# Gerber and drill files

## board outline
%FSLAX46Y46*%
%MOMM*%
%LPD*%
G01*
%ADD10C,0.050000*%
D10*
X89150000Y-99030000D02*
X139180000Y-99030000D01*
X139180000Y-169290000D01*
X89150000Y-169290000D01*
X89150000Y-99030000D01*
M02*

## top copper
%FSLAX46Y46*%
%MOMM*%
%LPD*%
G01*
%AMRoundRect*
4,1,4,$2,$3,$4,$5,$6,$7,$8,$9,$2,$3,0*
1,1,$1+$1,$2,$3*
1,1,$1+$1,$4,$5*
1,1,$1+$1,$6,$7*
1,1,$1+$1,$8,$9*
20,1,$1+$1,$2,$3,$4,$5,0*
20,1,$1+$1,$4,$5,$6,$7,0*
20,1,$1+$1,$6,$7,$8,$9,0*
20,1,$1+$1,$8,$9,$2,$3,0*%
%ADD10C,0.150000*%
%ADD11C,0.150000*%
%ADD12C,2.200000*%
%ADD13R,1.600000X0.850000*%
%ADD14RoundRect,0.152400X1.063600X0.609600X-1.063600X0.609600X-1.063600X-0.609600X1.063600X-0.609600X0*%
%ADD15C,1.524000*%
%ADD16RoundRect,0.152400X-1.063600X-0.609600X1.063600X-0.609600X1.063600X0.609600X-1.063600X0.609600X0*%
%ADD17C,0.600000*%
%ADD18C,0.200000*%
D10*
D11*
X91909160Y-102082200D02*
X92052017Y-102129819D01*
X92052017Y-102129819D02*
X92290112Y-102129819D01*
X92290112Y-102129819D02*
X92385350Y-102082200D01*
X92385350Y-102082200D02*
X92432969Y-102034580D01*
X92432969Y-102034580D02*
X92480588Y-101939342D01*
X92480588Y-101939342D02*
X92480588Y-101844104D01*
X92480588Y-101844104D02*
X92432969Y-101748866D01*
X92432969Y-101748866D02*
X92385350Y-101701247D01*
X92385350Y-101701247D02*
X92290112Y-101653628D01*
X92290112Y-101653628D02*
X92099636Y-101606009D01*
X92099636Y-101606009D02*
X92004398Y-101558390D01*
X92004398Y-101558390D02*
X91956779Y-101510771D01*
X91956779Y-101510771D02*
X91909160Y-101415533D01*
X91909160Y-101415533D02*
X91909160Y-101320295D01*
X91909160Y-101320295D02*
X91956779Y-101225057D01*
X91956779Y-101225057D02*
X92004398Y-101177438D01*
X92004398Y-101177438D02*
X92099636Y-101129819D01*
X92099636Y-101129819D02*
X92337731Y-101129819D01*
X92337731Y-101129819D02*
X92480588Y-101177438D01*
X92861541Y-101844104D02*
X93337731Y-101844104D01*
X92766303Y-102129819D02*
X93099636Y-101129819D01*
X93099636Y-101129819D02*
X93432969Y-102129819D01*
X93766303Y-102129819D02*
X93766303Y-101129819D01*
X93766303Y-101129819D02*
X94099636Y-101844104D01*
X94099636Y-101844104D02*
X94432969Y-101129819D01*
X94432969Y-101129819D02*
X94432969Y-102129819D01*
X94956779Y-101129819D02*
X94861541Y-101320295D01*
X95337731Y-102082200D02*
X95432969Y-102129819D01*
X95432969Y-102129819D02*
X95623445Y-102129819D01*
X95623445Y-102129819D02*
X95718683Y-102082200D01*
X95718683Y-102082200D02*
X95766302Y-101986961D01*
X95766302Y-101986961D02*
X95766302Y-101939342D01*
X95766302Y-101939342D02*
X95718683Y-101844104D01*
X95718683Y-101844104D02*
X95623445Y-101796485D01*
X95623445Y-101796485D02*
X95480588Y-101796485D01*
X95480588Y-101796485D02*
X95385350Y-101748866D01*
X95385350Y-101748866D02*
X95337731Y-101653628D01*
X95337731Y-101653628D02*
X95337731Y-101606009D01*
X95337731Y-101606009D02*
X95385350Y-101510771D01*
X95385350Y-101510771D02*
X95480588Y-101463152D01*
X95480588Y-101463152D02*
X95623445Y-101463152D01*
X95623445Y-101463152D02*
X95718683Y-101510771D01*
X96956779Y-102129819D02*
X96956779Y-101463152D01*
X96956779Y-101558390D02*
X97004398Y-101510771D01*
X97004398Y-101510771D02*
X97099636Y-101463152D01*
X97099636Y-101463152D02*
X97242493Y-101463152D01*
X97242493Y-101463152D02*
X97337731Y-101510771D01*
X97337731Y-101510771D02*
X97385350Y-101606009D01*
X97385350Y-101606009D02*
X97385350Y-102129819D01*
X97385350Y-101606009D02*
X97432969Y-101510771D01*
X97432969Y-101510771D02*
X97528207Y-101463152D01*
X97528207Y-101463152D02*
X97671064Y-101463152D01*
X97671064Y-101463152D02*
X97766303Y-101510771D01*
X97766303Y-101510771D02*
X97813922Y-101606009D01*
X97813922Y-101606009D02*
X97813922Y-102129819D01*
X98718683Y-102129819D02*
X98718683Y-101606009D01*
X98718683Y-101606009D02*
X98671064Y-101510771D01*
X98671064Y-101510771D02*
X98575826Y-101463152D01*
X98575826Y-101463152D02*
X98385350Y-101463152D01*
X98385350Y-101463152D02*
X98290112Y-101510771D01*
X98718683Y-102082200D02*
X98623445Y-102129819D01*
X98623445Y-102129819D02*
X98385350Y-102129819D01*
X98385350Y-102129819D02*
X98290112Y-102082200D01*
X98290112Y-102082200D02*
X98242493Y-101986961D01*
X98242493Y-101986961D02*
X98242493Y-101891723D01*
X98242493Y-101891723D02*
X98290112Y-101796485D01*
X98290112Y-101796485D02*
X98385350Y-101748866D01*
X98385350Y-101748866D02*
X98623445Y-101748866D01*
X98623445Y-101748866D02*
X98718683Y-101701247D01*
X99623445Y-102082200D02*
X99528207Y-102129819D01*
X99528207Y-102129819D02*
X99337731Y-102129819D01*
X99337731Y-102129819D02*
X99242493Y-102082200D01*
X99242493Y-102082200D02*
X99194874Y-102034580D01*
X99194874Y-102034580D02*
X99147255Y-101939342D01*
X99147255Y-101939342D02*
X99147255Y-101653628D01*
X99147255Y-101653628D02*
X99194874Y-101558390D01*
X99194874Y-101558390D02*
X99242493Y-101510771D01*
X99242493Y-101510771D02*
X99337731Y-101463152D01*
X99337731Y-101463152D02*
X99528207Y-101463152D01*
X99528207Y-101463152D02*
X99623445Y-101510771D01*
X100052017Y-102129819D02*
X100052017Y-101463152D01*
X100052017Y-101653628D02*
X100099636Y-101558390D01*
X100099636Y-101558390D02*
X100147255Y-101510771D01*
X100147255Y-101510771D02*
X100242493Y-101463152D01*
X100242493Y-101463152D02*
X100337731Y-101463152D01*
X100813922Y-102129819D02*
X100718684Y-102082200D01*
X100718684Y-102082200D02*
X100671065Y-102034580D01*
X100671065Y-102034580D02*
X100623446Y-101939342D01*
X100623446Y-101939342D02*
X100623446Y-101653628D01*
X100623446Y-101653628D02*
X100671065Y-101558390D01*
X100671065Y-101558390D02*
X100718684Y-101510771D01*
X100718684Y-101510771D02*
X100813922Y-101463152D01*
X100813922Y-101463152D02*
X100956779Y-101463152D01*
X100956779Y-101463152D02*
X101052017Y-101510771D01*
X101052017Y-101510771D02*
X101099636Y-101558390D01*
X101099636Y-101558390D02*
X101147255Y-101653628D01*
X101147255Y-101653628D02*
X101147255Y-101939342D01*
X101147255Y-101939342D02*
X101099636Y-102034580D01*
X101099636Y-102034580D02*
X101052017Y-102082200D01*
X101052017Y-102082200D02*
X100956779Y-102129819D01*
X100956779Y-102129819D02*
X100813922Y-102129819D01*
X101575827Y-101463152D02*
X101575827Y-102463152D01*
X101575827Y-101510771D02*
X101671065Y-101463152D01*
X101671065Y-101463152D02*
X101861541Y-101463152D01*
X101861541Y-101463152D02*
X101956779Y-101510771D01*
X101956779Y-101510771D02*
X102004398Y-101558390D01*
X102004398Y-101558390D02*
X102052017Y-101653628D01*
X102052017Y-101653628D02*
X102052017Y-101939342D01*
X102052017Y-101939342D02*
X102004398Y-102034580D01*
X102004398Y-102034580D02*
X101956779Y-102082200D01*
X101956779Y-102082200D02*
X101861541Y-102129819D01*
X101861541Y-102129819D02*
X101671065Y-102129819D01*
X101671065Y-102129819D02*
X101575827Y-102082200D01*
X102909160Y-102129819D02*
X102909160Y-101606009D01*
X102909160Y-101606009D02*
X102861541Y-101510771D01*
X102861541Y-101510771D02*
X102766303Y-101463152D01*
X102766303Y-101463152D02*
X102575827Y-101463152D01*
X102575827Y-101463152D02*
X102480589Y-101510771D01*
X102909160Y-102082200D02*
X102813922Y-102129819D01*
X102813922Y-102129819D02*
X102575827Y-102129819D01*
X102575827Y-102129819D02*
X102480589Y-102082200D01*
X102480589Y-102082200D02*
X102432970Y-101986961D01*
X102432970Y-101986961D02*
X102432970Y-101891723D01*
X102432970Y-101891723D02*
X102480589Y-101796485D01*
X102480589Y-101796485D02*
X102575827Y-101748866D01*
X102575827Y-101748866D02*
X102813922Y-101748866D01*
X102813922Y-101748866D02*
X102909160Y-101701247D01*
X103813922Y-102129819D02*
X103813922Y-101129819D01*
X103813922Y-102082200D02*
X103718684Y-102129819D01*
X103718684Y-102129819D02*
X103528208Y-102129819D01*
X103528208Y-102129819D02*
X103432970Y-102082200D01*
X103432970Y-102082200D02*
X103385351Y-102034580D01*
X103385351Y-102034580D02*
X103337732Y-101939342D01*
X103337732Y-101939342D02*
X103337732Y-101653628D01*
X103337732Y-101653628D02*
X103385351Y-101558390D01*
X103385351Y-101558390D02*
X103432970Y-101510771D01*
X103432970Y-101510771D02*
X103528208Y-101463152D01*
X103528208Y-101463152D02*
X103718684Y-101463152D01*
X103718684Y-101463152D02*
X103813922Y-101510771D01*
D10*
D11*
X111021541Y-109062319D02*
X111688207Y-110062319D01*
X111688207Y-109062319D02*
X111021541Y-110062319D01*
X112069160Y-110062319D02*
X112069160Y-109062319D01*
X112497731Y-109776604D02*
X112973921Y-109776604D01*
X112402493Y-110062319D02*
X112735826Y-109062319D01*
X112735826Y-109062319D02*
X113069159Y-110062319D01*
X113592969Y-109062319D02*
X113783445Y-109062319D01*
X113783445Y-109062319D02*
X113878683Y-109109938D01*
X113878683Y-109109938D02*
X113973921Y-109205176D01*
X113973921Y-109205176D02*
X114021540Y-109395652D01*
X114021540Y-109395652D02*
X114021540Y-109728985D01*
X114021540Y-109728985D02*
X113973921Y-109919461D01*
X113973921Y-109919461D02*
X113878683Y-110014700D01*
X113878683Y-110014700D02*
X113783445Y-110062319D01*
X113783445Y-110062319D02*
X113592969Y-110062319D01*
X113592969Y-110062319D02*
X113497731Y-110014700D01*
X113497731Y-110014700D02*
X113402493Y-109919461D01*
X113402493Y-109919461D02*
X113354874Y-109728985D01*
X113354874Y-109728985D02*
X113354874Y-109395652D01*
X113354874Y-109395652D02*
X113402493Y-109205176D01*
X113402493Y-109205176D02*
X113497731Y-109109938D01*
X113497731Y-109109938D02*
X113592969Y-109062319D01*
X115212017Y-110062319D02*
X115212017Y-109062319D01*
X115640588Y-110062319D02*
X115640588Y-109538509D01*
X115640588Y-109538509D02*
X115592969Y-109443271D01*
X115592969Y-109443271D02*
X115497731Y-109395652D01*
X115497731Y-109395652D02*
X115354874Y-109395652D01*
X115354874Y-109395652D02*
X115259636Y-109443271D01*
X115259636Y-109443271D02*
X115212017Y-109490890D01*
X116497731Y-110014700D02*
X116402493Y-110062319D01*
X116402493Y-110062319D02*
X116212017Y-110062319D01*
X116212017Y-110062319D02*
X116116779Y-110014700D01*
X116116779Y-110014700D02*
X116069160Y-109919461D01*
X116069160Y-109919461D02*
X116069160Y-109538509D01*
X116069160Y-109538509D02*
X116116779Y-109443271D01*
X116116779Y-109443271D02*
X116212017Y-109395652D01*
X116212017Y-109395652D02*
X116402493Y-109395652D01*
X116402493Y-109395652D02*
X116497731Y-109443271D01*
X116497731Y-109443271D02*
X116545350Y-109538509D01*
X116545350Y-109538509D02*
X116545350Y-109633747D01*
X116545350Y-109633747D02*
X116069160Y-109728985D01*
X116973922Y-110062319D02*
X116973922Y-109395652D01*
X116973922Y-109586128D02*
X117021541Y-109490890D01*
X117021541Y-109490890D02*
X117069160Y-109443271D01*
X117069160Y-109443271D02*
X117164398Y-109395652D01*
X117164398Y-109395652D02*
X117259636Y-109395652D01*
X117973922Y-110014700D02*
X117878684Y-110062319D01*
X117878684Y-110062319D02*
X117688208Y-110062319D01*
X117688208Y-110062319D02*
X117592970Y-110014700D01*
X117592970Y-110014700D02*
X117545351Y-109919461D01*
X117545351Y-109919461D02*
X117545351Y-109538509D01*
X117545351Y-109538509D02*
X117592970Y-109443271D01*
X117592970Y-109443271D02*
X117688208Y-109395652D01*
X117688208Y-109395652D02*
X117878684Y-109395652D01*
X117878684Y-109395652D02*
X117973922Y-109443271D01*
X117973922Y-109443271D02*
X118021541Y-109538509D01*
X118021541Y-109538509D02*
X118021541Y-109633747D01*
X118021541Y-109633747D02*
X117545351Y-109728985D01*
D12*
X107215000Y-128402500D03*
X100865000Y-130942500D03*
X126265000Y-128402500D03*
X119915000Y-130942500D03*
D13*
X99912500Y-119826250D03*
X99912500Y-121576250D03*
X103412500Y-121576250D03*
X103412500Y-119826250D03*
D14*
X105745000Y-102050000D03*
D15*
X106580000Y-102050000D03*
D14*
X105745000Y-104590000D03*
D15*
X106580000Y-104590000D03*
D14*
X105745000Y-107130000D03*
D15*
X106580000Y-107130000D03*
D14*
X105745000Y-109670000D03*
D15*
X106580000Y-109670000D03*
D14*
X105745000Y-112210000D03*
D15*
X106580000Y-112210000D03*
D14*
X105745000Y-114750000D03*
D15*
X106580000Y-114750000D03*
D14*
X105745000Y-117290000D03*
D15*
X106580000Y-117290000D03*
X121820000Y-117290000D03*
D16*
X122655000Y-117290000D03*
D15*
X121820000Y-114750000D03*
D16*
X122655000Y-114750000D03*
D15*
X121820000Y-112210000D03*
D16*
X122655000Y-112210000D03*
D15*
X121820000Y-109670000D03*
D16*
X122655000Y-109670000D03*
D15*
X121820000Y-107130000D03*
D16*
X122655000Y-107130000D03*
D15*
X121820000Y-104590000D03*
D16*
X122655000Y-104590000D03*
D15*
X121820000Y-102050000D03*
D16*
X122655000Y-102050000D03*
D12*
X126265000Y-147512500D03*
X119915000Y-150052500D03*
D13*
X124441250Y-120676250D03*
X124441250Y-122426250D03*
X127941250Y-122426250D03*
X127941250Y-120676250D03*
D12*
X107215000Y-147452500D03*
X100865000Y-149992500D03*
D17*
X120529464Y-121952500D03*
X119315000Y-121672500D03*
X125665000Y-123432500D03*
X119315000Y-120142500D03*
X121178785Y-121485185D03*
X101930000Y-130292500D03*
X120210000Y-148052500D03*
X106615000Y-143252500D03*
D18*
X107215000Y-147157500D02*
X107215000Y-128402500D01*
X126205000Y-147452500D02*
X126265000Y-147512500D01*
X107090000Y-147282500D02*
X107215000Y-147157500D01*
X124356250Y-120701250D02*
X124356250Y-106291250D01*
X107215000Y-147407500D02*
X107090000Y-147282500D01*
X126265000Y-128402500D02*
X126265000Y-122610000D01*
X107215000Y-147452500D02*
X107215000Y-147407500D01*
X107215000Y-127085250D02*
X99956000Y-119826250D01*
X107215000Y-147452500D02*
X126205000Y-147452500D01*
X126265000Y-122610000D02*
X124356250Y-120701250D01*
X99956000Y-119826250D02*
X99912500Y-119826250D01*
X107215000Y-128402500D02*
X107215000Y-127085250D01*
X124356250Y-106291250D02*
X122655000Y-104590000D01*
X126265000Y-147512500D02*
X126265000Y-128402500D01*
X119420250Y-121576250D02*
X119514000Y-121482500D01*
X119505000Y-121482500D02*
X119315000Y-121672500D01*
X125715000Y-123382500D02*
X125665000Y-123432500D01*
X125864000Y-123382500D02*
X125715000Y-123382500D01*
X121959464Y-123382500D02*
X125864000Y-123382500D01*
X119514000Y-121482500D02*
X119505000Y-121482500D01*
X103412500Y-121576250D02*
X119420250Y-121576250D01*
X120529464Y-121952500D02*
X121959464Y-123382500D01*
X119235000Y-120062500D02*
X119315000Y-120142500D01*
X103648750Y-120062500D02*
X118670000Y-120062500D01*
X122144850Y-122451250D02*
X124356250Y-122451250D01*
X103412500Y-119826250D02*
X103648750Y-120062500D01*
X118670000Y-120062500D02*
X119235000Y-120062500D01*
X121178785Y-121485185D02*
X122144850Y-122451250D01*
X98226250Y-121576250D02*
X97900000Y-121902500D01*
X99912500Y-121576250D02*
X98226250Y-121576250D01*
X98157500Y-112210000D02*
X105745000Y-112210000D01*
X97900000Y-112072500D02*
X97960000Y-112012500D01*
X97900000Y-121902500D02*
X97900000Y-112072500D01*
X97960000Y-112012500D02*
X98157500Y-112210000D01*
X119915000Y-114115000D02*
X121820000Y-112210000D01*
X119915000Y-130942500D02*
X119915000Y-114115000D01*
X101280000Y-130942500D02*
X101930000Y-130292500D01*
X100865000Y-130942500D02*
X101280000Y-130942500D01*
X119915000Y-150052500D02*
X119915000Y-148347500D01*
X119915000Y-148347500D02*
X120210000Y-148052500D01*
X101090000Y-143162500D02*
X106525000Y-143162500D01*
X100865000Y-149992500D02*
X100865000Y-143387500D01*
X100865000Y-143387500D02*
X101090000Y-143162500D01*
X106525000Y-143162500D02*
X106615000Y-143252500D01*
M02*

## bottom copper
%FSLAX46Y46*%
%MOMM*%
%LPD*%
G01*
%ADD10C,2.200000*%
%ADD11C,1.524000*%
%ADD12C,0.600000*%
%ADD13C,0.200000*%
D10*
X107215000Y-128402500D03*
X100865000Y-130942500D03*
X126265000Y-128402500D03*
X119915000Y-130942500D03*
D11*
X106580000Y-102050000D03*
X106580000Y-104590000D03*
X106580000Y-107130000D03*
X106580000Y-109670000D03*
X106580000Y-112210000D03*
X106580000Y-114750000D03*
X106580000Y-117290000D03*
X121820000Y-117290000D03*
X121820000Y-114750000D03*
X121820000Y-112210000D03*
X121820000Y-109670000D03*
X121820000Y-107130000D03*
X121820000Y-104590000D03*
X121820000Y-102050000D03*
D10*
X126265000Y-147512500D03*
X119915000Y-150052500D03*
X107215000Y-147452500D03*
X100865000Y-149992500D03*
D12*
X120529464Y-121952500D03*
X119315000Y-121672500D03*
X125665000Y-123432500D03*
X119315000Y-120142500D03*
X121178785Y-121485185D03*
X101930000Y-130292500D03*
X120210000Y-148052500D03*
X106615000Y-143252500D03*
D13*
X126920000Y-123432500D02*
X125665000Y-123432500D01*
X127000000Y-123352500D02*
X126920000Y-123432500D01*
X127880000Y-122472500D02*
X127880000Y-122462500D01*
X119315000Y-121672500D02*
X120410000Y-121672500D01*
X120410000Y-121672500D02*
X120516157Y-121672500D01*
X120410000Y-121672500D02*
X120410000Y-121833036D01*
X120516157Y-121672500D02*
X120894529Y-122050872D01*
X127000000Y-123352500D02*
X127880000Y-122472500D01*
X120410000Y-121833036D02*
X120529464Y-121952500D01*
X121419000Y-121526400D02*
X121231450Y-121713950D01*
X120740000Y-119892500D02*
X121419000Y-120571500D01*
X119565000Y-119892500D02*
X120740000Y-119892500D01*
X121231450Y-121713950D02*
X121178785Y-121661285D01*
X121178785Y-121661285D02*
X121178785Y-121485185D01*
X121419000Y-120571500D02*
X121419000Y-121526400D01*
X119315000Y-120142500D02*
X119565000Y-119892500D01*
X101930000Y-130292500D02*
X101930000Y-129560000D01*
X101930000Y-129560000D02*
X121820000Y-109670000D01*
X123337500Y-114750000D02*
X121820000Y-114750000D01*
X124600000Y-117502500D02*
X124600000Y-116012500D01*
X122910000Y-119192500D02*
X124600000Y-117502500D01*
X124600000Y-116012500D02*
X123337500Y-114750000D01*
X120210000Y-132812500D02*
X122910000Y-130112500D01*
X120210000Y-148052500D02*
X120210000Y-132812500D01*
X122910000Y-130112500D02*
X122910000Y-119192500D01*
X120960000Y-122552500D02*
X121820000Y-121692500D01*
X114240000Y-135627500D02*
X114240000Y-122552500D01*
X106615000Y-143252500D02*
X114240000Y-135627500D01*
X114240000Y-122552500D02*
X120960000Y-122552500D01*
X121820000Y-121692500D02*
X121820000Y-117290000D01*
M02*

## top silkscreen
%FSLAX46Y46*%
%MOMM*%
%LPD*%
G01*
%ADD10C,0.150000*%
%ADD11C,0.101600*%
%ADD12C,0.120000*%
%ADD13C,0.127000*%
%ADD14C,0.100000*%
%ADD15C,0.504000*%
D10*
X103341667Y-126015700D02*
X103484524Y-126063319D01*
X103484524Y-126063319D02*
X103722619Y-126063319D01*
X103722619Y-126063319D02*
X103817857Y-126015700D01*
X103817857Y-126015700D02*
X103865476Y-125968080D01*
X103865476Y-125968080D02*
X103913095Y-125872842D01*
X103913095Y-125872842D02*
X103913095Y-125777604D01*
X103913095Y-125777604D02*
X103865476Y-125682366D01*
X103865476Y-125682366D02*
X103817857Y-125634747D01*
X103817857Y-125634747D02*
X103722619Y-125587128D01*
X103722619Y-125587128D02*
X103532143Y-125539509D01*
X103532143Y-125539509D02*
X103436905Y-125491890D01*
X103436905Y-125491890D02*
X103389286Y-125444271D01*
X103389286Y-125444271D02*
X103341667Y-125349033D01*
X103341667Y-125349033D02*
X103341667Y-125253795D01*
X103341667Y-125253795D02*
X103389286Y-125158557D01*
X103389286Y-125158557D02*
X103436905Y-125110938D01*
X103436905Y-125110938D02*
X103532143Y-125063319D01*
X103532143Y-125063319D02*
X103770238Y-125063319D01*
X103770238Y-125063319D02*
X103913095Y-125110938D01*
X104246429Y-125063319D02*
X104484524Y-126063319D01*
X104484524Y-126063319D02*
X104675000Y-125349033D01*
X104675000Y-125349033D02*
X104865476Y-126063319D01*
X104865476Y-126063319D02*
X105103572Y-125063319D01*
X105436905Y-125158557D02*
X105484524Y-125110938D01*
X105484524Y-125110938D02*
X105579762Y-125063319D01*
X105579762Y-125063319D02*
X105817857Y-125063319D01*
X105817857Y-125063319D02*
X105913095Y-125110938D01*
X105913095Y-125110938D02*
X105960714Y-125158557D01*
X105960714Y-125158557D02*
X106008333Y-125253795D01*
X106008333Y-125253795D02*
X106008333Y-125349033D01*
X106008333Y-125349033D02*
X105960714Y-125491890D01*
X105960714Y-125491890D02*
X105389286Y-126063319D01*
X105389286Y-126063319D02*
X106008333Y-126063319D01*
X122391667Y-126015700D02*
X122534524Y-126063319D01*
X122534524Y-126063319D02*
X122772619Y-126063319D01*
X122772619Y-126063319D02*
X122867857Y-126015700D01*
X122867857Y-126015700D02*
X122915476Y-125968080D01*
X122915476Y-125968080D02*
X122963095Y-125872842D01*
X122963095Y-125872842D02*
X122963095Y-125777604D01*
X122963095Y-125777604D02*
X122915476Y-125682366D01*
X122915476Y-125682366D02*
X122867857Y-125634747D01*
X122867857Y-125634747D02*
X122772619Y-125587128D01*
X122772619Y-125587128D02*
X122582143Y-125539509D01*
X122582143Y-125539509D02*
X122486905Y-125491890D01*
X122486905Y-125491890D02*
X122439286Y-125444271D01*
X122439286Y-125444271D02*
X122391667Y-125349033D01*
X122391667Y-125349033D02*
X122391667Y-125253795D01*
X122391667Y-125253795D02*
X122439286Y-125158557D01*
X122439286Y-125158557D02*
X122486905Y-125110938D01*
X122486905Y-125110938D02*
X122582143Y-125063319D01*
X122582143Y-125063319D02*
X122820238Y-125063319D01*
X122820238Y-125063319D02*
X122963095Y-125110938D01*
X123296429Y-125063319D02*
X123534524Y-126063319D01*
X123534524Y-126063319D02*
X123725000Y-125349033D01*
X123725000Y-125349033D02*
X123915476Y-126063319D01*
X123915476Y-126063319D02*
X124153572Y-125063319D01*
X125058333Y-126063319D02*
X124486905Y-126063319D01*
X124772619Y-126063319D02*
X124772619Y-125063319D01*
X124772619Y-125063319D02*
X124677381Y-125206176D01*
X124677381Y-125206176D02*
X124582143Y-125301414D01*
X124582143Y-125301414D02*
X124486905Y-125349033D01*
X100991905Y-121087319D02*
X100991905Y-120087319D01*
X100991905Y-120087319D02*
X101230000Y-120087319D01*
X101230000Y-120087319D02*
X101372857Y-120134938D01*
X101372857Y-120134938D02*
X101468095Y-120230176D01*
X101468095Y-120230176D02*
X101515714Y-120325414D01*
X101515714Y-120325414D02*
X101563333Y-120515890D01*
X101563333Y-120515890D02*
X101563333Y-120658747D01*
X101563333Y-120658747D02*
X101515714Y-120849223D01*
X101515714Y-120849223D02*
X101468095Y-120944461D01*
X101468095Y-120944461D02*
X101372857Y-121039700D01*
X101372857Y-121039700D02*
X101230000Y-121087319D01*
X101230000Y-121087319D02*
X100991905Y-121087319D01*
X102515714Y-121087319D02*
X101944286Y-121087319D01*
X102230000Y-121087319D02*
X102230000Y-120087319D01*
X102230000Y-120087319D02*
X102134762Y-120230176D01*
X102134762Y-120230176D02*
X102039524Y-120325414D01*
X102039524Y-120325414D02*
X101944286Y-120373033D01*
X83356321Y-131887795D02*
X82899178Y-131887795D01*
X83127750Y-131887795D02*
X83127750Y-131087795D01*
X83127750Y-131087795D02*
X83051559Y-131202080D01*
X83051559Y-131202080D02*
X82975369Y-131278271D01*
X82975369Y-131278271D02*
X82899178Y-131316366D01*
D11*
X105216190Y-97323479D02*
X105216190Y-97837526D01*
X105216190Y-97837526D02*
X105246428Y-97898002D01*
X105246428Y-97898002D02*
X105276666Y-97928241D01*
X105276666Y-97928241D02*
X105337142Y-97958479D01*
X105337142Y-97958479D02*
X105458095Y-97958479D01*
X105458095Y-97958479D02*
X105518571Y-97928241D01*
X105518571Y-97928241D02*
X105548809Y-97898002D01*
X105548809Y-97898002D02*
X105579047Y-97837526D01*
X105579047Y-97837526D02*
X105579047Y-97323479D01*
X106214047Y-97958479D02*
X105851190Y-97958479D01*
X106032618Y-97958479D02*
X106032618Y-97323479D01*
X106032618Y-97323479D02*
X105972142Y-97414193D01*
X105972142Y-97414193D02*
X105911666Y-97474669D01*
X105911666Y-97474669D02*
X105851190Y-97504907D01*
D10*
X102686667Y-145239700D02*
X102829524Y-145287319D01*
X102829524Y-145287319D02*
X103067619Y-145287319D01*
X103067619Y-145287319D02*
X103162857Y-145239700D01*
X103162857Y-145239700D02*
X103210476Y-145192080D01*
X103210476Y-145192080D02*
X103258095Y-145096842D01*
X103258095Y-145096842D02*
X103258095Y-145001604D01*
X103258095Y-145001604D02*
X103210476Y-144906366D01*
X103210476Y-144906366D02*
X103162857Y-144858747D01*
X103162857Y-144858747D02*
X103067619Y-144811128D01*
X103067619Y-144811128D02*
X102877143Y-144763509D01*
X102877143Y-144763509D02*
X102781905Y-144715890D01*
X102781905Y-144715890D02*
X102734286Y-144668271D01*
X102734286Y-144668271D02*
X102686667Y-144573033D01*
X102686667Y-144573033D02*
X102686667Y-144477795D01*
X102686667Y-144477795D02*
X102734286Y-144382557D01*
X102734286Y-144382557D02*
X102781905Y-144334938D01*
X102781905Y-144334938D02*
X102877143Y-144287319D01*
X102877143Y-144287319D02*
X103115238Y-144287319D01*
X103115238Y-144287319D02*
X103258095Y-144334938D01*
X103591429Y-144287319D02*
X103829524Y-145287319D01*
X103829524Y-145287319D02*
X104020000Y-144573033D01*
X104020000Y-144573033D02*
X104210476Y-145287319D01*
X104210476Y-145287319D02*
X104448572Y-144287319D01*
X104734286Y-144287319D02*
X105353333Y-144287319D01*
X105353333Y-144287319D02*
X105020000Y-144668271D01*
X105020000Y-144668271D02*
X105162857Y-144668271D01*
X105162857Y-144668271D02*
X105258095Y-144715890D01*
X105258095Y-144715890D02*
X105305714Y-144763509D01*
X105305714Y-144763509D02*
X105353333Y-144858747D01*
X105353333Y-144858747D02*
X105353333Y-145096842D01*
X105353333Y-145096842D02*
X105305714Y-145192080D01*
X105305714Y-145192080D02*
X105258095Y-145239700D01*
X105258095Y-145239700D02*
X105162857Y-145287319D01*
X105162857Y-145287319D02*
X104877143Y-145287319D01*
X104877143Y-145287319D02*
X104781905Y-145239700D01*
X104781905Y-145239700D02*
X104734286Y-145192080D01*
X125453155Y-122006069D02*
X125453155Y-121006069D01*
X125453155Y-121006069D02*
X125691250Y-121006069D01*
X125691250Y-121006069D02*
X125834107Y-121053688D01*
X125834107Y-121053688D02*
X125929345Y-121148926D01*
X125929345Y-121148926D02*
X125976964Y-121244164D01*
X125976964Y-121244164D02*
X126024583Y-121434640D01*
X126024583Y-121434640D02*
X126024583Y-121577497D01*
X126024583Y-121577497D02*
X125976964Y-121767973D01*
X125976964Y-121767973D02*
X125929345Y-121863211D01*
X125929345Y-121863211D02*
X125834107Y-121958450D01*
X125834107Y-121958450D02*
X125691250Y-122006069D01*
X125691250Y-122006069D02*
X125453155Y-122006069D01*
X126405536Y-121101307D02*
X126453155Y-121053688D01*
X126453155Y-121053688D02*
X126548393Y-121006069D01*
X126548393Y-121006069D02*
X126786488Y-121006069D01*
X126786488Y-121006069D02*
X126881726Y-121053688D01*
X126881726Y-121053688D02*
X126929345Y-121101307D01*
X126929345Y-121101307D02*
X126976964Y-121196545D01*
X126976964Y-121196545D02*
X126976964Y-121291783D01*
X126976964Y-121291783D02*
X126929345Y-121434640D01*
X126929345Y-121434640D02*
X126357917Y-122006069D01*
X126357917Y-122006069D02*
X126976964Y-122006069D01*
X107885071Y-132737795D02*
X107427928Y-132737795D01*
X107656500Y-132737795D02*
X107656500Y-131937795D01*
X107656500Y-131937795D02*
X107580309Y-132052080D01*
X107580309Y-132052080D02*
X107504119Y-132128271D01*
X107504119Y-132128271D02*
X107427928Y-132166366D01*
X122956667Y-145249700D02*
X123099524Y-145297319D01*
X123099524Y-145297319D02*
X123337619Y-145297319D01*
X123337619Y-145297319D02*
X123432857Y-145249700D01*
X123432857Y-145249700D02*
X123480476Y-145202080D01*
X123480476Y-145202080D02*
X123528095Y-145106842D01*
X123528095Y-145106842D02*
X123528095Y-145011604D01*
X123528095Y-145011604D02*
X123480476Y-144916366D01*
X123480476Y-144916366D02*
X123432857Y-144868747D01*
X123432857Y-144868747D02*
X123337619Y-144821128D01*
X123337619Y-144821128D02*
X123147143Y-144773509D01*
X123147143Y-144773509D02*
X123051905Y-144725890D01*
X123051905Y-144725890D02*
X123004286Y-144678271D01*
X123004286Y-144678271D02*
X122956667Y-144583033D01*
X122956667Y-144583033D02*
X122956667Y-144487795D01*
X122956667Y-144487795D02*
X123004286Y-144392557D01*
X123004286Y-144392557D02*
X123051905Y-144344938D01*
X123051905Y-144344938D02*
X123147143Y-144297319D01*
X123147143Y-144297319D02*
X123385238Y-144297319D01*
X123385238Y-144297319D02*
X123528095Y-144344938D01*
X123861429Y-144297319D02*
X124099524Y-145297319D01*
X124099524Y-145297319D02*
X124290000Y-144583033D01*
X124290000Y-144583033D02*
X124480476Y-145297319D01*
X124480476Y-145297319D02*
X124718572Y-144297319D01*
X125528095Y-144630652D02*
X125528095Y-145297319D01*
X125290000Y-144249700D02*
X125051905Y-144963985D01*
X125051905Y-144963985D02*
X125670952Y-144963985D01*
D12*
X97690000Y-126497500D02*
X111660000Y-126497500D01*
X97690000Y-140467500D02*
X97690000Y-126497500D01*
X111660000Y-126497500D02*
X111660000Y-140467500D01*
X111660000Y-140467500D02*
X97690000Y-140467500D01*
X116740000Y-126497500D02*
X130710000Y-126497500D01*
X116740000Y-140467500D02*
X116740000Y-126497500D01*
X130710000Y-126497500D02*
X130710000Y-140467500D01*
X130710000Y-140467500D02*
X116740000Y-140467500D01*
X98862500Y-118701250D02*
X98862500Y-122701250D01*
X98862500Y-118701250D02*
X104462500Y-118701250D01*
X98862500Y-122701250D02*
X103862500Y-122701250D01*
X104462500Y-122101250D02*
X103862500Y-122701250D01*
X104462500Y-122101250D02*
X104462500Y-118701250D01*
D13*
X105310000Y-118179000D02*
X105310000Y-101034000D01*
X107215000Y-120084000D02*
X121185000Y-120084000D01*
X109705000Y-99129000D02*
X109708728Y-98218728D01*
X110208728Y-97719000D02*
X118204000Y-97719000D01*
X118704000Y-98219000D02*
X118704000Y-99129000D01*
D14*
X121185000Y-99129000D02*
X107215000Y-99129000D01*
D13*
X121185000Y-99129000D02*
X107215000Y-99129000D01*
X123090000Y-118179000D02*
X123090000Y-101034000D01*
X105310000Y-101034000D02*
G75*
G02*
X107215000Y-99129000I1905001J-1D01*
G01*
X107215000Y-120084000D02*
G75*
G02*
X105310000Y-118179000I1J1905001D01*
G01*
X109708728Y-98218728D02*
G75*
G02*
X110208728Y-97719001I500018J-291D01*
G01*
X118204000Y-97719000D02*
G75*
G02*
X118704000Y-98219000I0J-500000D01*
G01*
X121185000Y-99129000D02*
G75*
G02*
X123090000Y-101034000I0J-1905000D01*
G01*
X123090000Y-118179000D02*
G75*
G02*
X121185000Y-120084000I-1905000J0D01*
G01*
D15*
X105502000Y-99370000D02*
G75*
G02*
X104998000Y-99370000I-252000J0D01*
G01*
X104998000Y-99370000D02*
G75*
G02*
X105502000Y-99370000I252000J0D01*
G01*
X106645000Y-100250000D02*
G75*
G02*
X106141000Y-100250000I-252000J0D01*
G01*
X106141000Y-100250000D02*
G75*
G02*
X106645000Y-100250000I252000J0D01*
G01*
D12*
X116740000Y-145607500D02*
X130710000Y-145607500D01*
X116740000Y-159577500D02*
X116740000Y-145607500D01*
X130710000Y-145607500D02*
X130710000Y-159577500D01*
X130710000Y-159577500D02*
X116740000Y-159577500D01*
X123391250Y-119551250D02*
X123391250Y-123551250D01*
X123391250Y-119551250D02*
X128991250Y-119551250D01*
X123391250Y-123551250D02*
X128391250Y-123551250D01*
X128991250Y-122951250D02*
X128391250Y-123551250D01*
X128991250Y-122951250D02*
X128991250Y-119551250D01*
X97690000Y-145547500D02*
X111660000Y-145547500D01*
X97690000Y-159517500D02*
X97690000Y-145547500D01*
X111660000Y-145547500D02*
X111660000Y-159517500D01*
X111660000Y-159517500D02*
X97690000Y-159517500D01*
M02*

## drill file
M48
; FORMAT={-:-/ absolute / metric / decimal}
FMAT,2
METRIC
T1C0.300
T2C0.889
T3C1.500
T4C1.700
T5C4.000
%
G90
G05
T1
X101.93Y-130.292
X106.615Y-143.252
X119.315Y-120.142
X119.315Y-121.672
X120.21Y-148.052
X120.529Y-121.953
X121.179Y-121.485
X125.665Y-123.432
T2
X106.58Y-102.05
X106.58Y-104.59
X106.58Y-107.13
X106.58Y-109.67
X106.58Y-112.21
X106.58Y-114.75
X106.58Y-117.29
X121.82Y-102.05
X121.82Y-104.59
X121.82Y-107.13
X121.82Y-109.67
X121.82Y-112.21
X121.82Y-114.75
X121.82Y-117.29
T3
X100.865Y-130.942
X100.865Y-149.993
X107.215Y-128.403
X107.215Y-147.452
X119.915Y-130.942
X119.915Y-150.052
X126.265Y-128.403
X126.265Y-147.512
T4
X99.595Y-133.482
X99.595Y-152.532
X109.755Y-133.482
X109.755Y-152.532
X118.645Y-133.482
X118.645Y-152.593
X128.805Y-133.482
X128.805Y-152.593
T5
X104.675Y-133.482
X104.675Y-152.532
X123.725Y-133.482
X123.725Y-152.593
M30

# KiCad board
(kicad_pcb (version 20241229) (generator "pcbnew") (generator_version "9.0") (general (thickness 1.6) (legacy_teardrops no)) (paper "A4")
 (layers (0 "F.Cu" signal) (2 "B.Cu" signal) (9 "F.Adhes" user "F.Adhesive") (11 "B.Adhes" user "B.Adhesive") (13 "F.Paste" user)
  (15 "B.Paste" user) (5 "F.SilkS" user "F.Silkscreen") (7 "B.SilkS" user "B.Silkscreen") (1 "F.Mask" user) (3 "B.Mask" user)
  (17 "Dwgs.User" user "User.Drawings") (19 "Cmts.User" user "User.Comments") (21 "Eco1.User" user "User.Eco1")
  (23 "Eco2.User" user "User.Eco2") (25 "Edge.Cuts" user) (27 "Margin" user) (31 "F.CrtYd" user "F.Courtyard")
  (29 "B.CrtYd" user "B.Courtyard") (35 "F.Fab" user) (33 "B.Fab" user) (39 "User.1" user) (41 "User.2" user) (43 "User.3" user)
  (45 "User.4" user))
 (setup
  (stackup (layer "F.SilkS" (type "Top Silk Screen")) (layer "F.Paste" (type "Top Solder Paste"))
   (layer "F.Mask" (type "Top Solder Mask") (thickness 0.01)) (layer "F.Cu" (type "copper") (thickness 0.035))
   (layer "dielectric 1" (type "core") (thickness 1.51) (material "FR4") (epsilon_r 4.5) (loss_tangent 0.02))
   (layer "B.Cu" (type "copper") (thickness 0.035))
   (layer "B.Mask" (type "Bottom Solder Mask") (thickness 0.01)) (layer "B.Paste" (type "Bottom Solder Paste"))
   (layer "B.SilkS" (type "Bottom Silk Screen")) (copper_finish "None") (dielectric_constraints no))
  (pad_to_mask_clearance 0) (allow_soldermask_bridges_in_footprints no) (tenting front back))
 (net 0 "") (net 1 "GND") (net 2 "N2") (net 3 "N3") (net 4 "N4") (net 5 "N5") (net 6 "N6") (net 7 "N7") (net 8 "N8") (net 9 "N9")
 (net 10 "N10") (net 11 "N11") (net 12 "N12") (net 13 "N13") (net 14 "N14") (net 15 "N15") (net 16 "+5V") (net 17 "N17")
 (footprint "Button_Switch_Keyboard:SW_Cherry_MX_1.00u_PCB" (layer "F.Cu") (at 107.215 128.4025)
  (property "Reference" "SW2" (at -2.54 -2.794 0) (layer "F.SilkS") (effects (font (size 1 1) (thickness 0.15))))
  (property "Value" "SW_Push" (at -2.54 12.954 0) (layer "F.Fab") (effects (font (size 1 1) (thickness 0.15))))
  (fp_line (start -9.525 -1.905) (end 4.445 -1.905) (stroke (width 0.12) (type solid)) (layer "F.SilkS"))
  (fp_line (start -9.525 12.065) (end -9.525 -1.905) (stroke (width 0.12) (type solid)) (layer "F.SilkS"))
  (fp_line (start 4.445 -1.905) (end 4.445 12.065) (stroke (width 0.12) (type solid)) (layer "F.SilkS"))
  (fp_line (start 4.445 12.065) (end -9.525 12.065) (stroke (width 0.12) (type solid)) (layer "F.SilkS"))
  (pad "" np_thru_hole circle (at -7.62 5.08) (size 1.7 1.7) (drill 1.7) (layers "*.Cu" "*.Mask"))
  (pad "" np_thru_hole circle (at -2.54 5.08) (size 4 4) (drill 4) (layers "*.Cu" "*.Mask"))
  (pad "" np_thru_hole circle (at 2.54 5.08) (size 1.7 1.7) (drill 1.7) (layers "*.Cu" "*.Mask"))
  (pad "1" thru_hole circle (at 0 0) (size 2.2 2.2) (drill 1.5) (layers "*.Cu" "*.Mask") (remove_unused_layers no) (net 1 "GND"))
  (pad "2" thru_hole circle (at -6.35 2.54) (size 2.2 2.2) (drill 1.5) (layers "*.Cu" "*.Mask") (remove_unused_layers no) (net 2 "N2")))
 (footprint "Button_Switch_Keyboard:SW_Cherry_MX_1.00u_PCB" (layer "F.Cu") (at 126.265 128.4025)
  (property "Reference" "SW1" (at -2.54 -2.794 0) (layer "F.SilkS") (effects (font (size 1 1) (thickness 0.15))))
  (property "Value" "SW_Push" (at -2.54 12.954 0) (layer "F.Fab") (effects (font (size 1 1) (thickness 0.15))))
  (fp_line (start -9.525 -1.905) (end 4.445 -1.905) (stroke (width 0.12) (type solid)) (layer "F.SilkS"))
  (fp_line (start -9.525 12.065) (end -9.525 -1.905) (stroke (width 0.12) (type solid)) (layer "F.SilkS"))
  (fp_line (start 4.445 -1.905) (end 4.445 12.065) (stroke (width 0.12) (type solid)) (layer "F.SilkS"))
  (fp_line (start 4.445 12.065) (end -9.525 12.065) (stroke (width 0.12) (type solid)) (layer "F.SilkS"))
  (pad "" np_thru_hole circle (at -7.62 5.08) (size 1.7 1.7) (drill 1.7) (layers "*.Cu" "*.Mask"))
  (pad "" np_thru_hole circle (at -2.54 5.08) (size 4 4) (drill 4) (layers "*.Cu" "*.Mask"))
  (pad "" np_thru_hole circle (at 2.54 5.08) (size 1.7 1.7) (drill 1.7) (layers "*.Cu" "*.Mask"))
  (pad "1" thru_hole circle (at 0 0) (size 2.2 2.2) (drill 1.5) (layers "*.Cu" "*.Mask") (remove_unused_layers no) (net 1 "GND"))
  (pad "2" thru_hole circle (at -6.35 2.54) (size 2.2 2.2) (drill 1.5) (layers "*.Cu" "*.Mask") (remove_unused_layers no) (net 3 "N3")))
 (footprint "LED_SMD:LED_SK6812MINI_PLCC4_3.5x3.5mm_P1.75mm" (layer "F.Cu") (at 101.6625 120.70125)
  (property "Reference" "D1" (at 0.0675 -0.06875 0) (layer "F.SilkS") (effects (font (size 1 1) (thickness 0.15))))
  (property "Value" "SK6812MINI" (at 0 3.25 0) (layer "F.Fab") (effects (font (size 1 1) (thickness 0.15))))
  (fp_line (start -2.8 -2) (end -2.8 2) (stroke (width 0.12) (type default)) (layer "F.SilkS"))
  (fp_line (start -2.8 -2) (end 2.8 -2) (stroke (width 0.12) (type solid)) (layer "F.SilkS"))
  (fp_line (start -2.8 2) (end 2.2 2) (stroke (width 0.12) (type solid)) (layer "F.SilkS"))
  (fp_line (start 2.8 1.4) (end 2.2 2) (stroke (width 0.12) (type default)) (layer "F.SilkS"))
  (fp_line (start 2.8 1.4) (end 2.8 -2) (stroke (width 0.12) (type solid)) (layer "F.SilkS"))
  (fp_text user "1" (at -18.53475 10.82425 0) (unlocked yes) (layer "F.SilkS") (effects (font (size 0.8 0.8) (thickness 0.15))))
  (pad "1" smd rect (at -1.75 -0.875) (size 1.6 0.85) (layers "F.Cu" "F.Mask" "F.Paste") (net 1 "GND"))
  (pad "2" smd rect (at -1.75 0.875) (size 1.6 0.85) (layers "F.Cu" "F.Mask" "F.Paste") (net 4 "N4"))
  (pad "3" smd rect (at 1.75 0.875) (size 1.6 0.85) (layers "F.Cu" "F.Mask" "F.Paste") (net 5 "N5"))
  (pad "4" smd rect (at 1.75 -0.875) (size 1.6 0.85) (layers "F.Cu" "F.Mask" "F.Paste") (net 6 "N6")))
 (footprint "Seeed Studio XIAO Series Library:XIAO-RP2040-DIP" (layer "F.Cu") (at 114.2 109.67)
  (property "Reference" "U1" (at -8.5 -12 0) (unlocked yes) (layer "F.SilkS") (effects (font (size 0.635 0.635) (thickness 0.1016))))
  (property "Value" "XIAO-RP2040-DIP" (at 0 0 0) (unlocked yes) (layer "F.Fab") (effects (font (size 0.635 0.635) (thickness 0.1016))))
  (fp_line (start -8.89 8.509) (end -8.89 -8.636) (stroke (width 0.127) (type solid)) (layer "F.SilkS"))
  (fp_line (start -6.985 10.414) (end 6.985 10.414) (stroke (width 0.127) (type solid)) (layer "F.SilkS"))
  (fp_line (start -4.495 -10.541) (end -4.491272 -11.451272) (stroke (width 0.127) (type solid)) (layer "F.SilkS"))
  (fp_line (start -3.991272 -11.951) (end 4.004 -11.951) (stroke (width 0.127) (type solid)) (layer "F.SilkS"))
  (fp_line (start 4.504 -11.451) (end 4.504 -10.541) (stroke (width 0.127) (type solid)) (layer "F.SilkS"))
  (fp_line (start 6.985 -10.541) (end -6.985 -10.541) (stroke (width 0.1) (type solid)) (layer "F.SilkS"))
  (fp_line (start 6.985 -10.541) (end -6.985 -10.541) (stroke (width 0.127) (type solid)) (layer "F.SilkS"))
  (fp_line (start 8.89 8.509) (end 8.89 -8.636) (stroke (width 0.127) (type solid)) (layer "F.SilkS"))
  (fp_arc (start -8.89 -8.636) (mid -8.332038 -9.983038) (end -6.985 -10.541) (stroke (width 0.127) (type solid)) (layer "F.SilkS"))
  (fp_arc (start -6.985 10.414) (mid -8.332038 9.856038) (end -8.89 8.509) (stroke (width 0.127) (type solid)) (layer "F.SilkS"))
  (fp_arc (start -4.491272 -11.451272) (mid -4.344728 -11.80464) (end -3.991272 -11.951) (stroke (width 0.127) (type default))
   (layer "F.SilkS"))
  (fp_arc (start 4.004 -11.951) (mid 4.357553 -11.804553) (end 4.504 -11.451) (stroke (width 0.127) (type default)) (layer "F.SilkS"))
  (fp_arc (start 6.985 -10.541) (mid 8.332038 -9.983038) (end 8.89 -8.636) (stroke (width 0.127) (type solid)) (layer "F.SilkS"))
  (fp_arc (start 8.89 8.509) (mid 8.332038 9.856038) (end 6.985 10.414) (stroke (width 0.127) (type solid)) (layer "F.SilkS"))
  (fp_circle (center -8.95 -10.3) (end -8.95 -10.554) (stroke (width 0.5) (type solid)) (fill yes) (layer "F.SilkS"))
  (fp_circle (center -7.807 -9.42) (end -7.807 -9.674) (stroke (width 0.5) (type solid)) (fill yes) (layer "F.SilkS"))
  (pad "1" smd roundrect (at -8.455 -7.62 180) (size 2.432 1.524) (layers "F.Cu" "F.Mask") (roundrect_rratio 0.1) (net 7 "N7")
   (thermal_bridge_angle 45))
  (pad "1" thru_hole circle (at -7.62 -7.62 180) (size 1.524 1.524) (drill 0.889) (layers "*.Cu" "*.Mask") (remove_unused_layers no)
   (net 7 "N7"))
  (pad "2" smd roundrect (at -8.455 -5.08 180) (size 2.432 1.524) (layers "F.Cu" "F.Mask") (roundrect_rratio 0.1) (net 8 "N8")
   (thermal_bridge_angle 45))
  (pad "2" thru_hole circle (at -7.62 -5.08 180) (size 1.524 1.524) (drill 0.889) (layers "*.Cu" "*.Mask") (remove_unused_layers no)
   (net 8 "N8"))
  (pad "3" smd roundrect (at -8.455 -2.54 180) (size 2.432 1.524) (layers "F.Cu" "F.Mask") (roundrect_rratio 0.1) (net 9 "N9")
   (thermal_bridge_angle 45))
  (pad "3" thru_hole circle (at -7.62 -2.54 180) (size 1.524 1.524) (drill 0.889) (layers "*.Cu" "*.Mask") (remove_unused_layers no)
   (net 9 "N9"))
  (pad "4" smd roundrect (at -8.455 0 180) (size 2.432 1.524) (layers "F.Cu" "F.Mask") (roundrect_rratio 0.1) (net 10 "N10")
   (thermal_bridge_angle 45))
  (pad "4" thru_hole circle (at -7.62 0 180) (size 1.524 1.524) (drill 0.889) (layers "*.Cu" "*.Mask") (remove_unused_layers no)
   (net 10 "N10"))
  (pad "5" smd roundrect (at -8.455 2.54 180) (size 2.432 1.524) (layers "F.Cu" "F.Mask") (roundrect_rratio 0.1) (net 4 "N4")
   (thermal_bridge_angle 45))
  (pad "5" thru_hole circle (at -7.62 2.54 180) (size 1.524 1.524) (drill 0.889) (layers "*.Cu" "*.Mask") (remove_unused_layers no)
   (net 4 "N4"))
  (pad "6" smd roundrect (at -8.455 5.08 180) (size 2.432 1.524) (layers "F.Cu" "F.Mask") (roundrect_rratio 0.1) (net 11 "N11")
   (thermal_bridge_angle 45))
  (pad "6" thru_hole circle (at -7.62 5.08 180) (size 1.524 1.524) (drill 0.889) (layers "*.Cu" "*.Mask") (remove_unused_layers no)
   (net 11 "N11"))
  (pad "7" smd roundrect (at -8.455 7.62 180) (size 2.432 1.524) (layers "F.Cu" "F.Mask") (roundrect_rratio 0.1) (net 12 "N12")
   (thermal_bridge_angle 45))
  (pad "7" thru_hole circle (at -7.62 7.62 180) (size 1.524 1.524) (drill 0.889) (layers "*.Cu" "*.Mask") (remove_unused_layers no)
   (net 12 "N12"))
  (pad "8" thru_hole circle (at 7.62 7.62) (size 1.524 1.524) (drill 0.889) (layers "*.Cu" "*.Mask") (remove_unused_layers no)
   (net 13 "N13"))
  (pad "8" smd roundrect (at 8.455 7.62) (size 2.432 1.524) (layers "F.Cu" "F.Mask") (roundrect_rratio 0.1) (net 13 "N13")
   (thermal_bridge_angle 45))
  (pad "9" thru_hole circle (at 7.62 5.08) (size 1.524 1.524) (drill 0.889) (layers "*.Cu" "*.Mask") (remove_unused_layers no)
   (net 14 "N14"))
  (pad "9" smd roundrect (at 8.455 5.08) (size 2.432 1.524) (layers "F.Cu" "F.Mask") (roundrect_rratio 0.1) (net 14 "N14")
   (thermal_bridge_angle 45))
  (pad "10" thru_hole circle (at 7.62 2.54) (size 1.524 1.524) (drill 0.889) (layers "*.Cu" "*.Mask") (remove_unused_layers no) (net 3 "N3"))
  (pad "10" smd roundrect (at 8.455 2.54) (size 2.432 1.524) (layers "F.Cu" "F.Mask") (roundrect_rratio 0.1) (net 3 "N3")
   (thermal_bridge_angle 45))
  (pad "11" thru_hole circle (at 7.62 0) (size 1.524 1.524) (drill 0.889) (layers "*.Cu" "*.Mask") (remove_unused_layers no) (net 2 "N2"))
  (pad "11" smd roundrect (at 8.455 0) (size 2.432 1.524) (layers "F.Cu" "F.Mask") (roundrect_rratio 0.1) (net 2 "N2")
   (thermal_bridge_angle 45))
  (pad "12" thru_hole circle (at 7.62 -2.54) (size 1.524 1.524) (drill 0.889) (layers "*.Cu" "*.Mask") (remove_unused_layers no)
   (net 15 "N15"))
  (pad "12" smd roundrect (at 8.455 -2.54) (size 2.432 1.524) (layers "F.Cu" "F.Mask") (roundrect_rratio 0.1) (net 15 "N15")
   (thermal_bridge_angle 45))
  (pad "13" thru_hole circle (at 7.62 -5.08) (size 1.524 1.524) (drill 0.889) (layers "*.Cu" "*.Mask") (remove_unused_layers no)
   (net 1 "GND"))
  (pad "13" smd roundrect (at 8.455 -5.08) (size 2.432 1.524) (layers "F.Cu" "F.Mask") (roundrect_rratio 0.1) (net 1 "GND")
   (thermal_bridge_angle 45))
  (pad "14" thru_hole circle (at 7.62 -7.62) (size 1.524 1.524) (drill 0.889) (layers "*.Cu" "*.Mask") (remove_unused_layers no)
   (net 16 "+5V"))
  (pad "14" smd roundrect (at 8.455 -7.62) (size 2.432 1.524) (layers "F.Cu" "F.Mask") (roundrect_rratio 0.1) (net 16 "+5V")
   (thermal_bridge_angle 45)))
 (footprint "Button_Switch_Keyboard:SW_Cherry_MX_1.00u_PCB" (layer "F.Cu") (at 126.265 147.5125)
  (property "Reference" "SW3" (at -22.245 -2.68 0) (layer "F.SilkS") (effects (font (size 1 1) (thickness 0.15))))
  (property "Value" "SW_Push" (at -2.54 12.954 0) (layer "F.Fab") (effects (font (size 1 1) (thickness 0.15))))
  (fp_line (start -9.525 -1.905) (end 4.445 -1.905) (stroke (width 0.12) (type solid)) (layer "F.SilkS"))
  (fp_line (start -9.525 12.065) (end -9.525 -1.905) (stroke (width 0.12) (type solid)) (layer "F.SilkS"))
  (fp_line (start 4.445 -1.905) (end 4.445 12.065) (stroke (width 0.12) (type solid)) (layer "F.SilkS"))
  (fp_line (start 4.445 12.065) (end -9.525 12.065) (stroke (width 0.12) (type solid)) (layer "F.SilkS"))
  (pad "" np_thru_hole circle (at -7.62 5.08) (size 1.7 1.7) (drill 1.7) (layers "*.Cu" "*.Mask"))
  (pad "" np_thru_hole circle (at -2.54 5.08) (size 4 4) (drill 4) (layers "*.Cu" "*.Mask"))
  (pad "" np_thru_hole circle (at 2.54 5.08) (size 1.7 1.7) (drill 1.7) (layers "*.Cu" "*.Mask"))
  (pad "1" thru_hole circle (at 0 0) (size 2.2 2.2) (drill 1.5) (layers "*.Cu" "*.Mask") (remove_unused_layers no) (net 1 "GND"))
  (pad "2" thru_hole circle (at -6.35 2.54) (size 2.2 2.2) (drill 1.5) (layers "*.Cu" "*.Mask") (remove_unused_layers no) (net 14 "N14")))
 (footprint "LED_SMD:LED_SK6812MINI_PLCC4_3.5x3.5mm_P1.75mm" (layer "F.Cu") (at 126.19125 121.55125)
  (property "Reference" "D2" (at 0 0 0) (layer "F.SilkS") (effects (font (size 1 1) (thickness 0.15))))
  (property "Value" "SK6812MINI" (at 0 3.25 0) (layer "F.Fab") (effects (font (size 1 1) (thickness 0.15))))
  (fp_line (start -2.8 -2) (end -2.8 2) (stroke (width 0.12) (type default)) (layer "F.SilkS"))
  (fp_line (start -2.8 -2) (end 2.8 -2) (stroke (width 0.12) (type solid)) (layer "F.SilkS"))
  (fp_line (start -2.8 2) (end 2.2 2) (stroke (width 0.12) (type solid)) (layer "F.SilkS"))
  (fp_line (start 2.8 1.4) (end 2.2 2) (stroke (width 0.12) (type default)) (layer "F.SilkS"))
  (fp_line (start 2.8 1.4) (end 2.8 -2) (stroke (width 0.12) (type solid)) (layer "F.SilkS"))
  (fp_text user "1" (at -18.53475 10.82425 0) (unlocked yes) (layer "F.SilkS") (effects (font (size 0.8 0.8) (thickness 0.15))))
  (pad "1" smd rect (at -1.75 -0.875) (size 1.6 0.85) (layers "F.Cu" "F.Mask" "F.Paste") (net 1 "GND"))
  (pad "2" smd rect (at -1.75 0.875) (size 1.6 0.85) (layers "F.Cu" "F.Mask" "F.Paste") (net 6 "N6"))
  (pad "3" smd rect (at 1.75 0.875) (size 1.6 0.85) (layers "F.Cu" "F.Mask" "F.Paste") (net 5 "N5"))
  (pad "4" smd rect (at 1.75 -0.875) (size 1.6 0.85) (layers "F.Cu" "F.Mask" "F.Paste") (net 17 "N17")))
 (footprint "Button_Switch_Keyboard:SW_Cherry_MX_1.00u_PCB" (layer "F.Cu") (at 107.215 147.4525)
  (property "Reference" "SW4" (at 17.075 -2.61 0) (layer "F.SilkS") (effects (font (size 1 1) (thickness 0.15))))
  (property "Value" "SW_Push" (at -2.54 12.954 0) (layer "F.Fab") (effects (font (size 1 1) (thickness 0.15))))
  (fp_line (start -9.525 -1.905) (end 4.445 -1.905) (stroke (width 0.12) (type solid)) (layer "F.SilkS"))
  (fp_line (start -9.525 12.065) (end -9.525 -1.905) (stroke (width 0.12) (type solid)) (layer "F.SilkS"))
  (fp_line (start 4.445 -1.905) (end 4.445 12.065) (stroke (width 0.12) (type solid)) (layer "F.SilkS"))
  (fp_line (start 4.445 12.065) (end -9.525 12.065) (stroke (width 0.12) (type solid)) (layer "F.SilkS"))
  (pad "" np_thru_hole circle (at -7.62 5.08) (size 1.7 1.7) (drill 1.7) (layers "*.Cu" "*.Mask"))
  (pad "" np_thru_hole circle (at -2.54 5.08) (size 4 4) (drill 4) (layers "*.Cu" "*.Mask"))
  (pad "" np_thru_hole circle (at 2.54 5.08) (size 1.7 1.7) (drill 1.7) (layers "*.Cu" "*.Mask"))
  (pad "1" thru_hole circle (at 0 0) (size 2.2 2.2) (drill 1.5) (layers "*.Cu" "*.Mask") (remove_unused_layers no) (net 1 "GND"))
  (pad "2" thru_hole circle (at -6.35 2.54) (size 2.2 2.2) (drill 1.5) (layers "*.Cu" "*.Mask") (remove_unused_layers no) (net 13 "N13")))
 (gr_rect (start 89.15 99.03) (end 139.18 169.29) (stroke (width 0.05) (type default)) (fill no) (layer "Edge.Cuts"))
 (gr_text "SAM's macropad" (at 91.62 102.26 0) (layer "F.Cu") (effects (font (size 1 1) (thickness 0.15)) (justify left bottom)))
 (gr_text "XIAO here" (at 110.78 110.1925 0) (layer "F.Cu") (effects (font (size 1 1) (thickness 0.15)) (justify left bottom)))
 (segment (start 107.215 147.1575) (end 107.215 128.4025) (width 0.2) (layer "F.Cu") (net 1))
 (segment (start 126.205 147.4525) (end 126.265 147.5125) (width 0.2) (layer "F.Cu") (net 1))
 (segment (start 107.09 147.2825) (end 107.215 147.1575) (width 0.2) (layer "F.Cu") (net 1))
 (segment (start 124.35625 120.70125) (end 124.35625 106.29125) (width 0.2) (layer "F.Cu") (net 1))
 (segment (start 107.215 147.4075) (end 107.09 147.2825) (width 0.2) (layer "F.Cu") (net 1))
 (segment (start 126.265 128.4025) (end 126.265 122.61) (width 0.2) (layer "F.Cu") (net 1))
 (segment (start 107.215 147.4525) (end 107.215 147.4075) (width 0.2) (layer "F.Cu") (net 1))
 (segment (start 107.215 127.08525) (end 99.956 119.82625) (width 0.2) (layer "F.Cu") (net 1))
 (segment (start 107.215 147.4525) (end 126.205 147.4525) (width 0.2) (layer "F.Cu") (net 1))
 (segment (start 126.265 122.61) (end 124.35625 120.70125) (width 0.2) (layer "F.Cu") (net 1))
 (segment (start 99.956 119.82625) (end 99.9125 119.82625) (width 0.2) (layer "F.Cu") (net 1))
 (segment (start 107.215 128.4025) (end 107.215 127.08525) (width 0.2) (layer "F.Cu") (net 1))
 (segment (start 124.35625 106.29125) (end 122.655 104.59) (width 0.2) (layer "F.Cu") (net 1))
 (segment (start 126.265 147.5125) (end 126.265 128.4025) (width 0.2) (layer "F.Cu") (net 1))
 (segment (start 119.42025 121.57625) (end 119.514 121.4825) (width 0.2) (layer "F.Cu") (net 5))
 (segment (start 119.505 121.4825) (end 119.315 121.6725) (width 0.2) (layer "F.Cu") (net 5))
 (segment (start 125.715 123.3825) (end 125.665 123.4325) (width 0.2) (layer "F.Cu") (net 5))
 (segment (start 125.864 123.3825) (end 125.715 123.3825) (width 0.2) (layer "F.Cu") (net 5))
 (segment (start 121.959464 123.3825) (end 125.864 123.3825) (width 0.2) (layer "F.Cu") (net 5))
 (segment (start 119.514 121.4825) (end 119.505 121.4825) (width 0.2) (layer "F.Cu") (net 5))
 (segment (start 103.4125 121.57625) (end 119.42025 121.57625) (width 0.2) (layer "F.Cu") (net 5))
 (segment (start 120.529464 121.9525) (end 121.959464 123.3825) (width 0.2) (layer "F.Cu") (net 5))
 (via (at 120.529464 121.9525) (size 0.6) (drill 0.3) (layers "F.Cu" "B.Cu") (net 5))
 (via (at 119.315 121.6725) (size 0.6) (drill 0.3) (layers "F.Cu" "B.Cu") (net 5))
 (via (at 125.665 123.4325) (size 0.6) (drill 0.3) (layers "F.Cu" "B.Cu") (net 5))
 (segment (start 126.92 123.4325) (end 125.665 123.4325) (width 0.2) (layer "B.Cu") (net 5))
 (segment (start 127 123.3525) (end 126.92 123.4325) (width 0.2) (layer "B.Cu") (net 5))
 (segment (start 127.88 122.4725) (end 127.88 122.4625) (width 0.2) (layer "B.Cu") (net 5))
 (segment (start 119.315 121.6725) (end 120.41 121.6725) (width 0.2) (layer "B.Cu") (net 5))
 (segment (start 120.41 121.6725) (end 120.516157 121.6725) (width 0.2) (layer "B.Cu") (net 5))
 (segment (start 120.41 121.6725) (end 120.41 121.833036) (width 0.2) (layer "B.Cu") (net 5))
 (segment (start 120.516157 121.6725) (end 120.894529 122.050872) (width 0.2) (layer "B.Cu") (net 5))
 (segment (start 127 123.3525) (end 127.88 122.4725) (width 0.2) (layer "B.Cu") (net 5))
 (segment (start 120.41 121.833036) (end 120.529464 121.9525) (width 0.2) (layer "B.Cu") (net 5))
 (segment (start 119.235 120.0625) (end 119.315 120.1425) (width 0.2) (layer "F.Cu") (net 6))
 (segment (start 103.64875 120.0625) (end 118.67 120.0625) (width 0.2) (layer "F.Cu") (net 6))
 (segment (start 122.14485 122.45125) (end 124.35625 122.45125) (width 0.2) (layer "F.Cu") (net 6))
 (segment (start 103.4125 119.82625) (end 103.64875 120.0625) (width 0.2) (layer "F.Cu") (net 6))
 (segment (start 118.67 120.0625) (end 119.235 120.0625) (width 0.2) (layer "F.Cu") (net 6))
 (segment (start 121.178785 121.485185) (end 122.14485 122.45125) (width 0.2) (layer "F.Cu") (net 6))
 (via (at 119.315 120.1425) (size 0.6) (drill 0.3) (layers "F.Cu" "B.Cu") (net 6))
 (via (at 121.178785 121.485185) (size 0.6) (drill 0.3) (layers "F.Cu" "B.Cu") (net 6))
 (segment (start 121.419 121.5264) (end 121.23145 121.71395) (width 0.2) (layer "B.Cu") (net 6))
 (segment (start 120.74 119.8925) (end 121.419 120.5715) (width 0.2) (layer "B.Cu") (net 6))
 (segment (start 119.565 119.8925) (end 120.74 119.8925) (width 0.2) (layer "B.Cu") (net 6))
 (segment (start 121.23145 121.71395) (end 121.178785 121.661285) (width 0.2) (layer "B.Cu") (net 6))
 (segment (start 121.178785 121.661285) (end 121.178785 121.485185) (width 0.2) (layer "B.Cu") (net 6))
 (segment (start 121.419 120.5715) (end 121.419 121.5264) (width 0.2) (layer "B.Cu") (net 6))
 (segment (start 119.315 120.1425) (end 119.565 119.8925) (width 0.2) (layer "B.Cu") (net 6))
 (segment (start 98.22625 121.57625) (end 97.9 121.9025) (width 0.2) (layer "F.Cu") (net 4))
 (segment (start 99.9125 121.57625) (end 98.22625 121.57625) (width 0.2) (layer "F.Cu") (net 4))
 (segment (start 98.1575 112.21) (end 105.745 112.21) (width 0.2) (layer "F.Cu") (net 4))
 (segment (start 97.9 112.0725) (end 97.96 112.0125) (width 0.2) (layer "F.Cu") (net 4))
 (segment (start 97.9 121.9025) (end 97.9 112.0725) (width 0.2) (layer "F.Cu") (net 4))
 (segment (start 97.96 112.0125) (end 98.1575 112.21) (width 0.2) (layer "F.Cu") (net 4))
 (segment (start 119.915 114.115) (end 121.82 112.21) (width 0.2) (layer "F.Cu") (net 3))
 (segment (start 119.915 130.9425) (end 119.915 114.115) (width 0.2) (layer "F.Cu") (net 3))
 (segment (start 101.28 130.9425) (end 101.93 130.2925) (width 0.2) (layer "F.Cu") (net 2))
 (segment (start 100.865 130.9425) (end 101.28 130.9425) (width 0.2) (layer "F.Cu") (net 2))
 (via (at 101.93 130.2925) (size 0.6) (drill 0.3) (layers "F.Cu" "B.Cu") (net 2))
 (segment (start 101.93 130.2925) (end 101.93 129.56) (width 0.2) (layer "B.Cu") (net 2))
 (segment (start 101.93 129.56) (end 121.82 109.67) (width 0.2) (layer "B.Cu") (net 2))
 (segment (start 119.915 150.0525) (end 119.915 148.3475) (width 0.2) (layer "F.Cu") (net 14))
 (segment (start 119.915 148.3475) (end 120.21 148.0525) (width 0.2) (layer "F.Cu") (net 14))
 (via (at 120.21 148.0525) (size 0.6) (drill 0.3) (layers "F.Cu" "B.Cu") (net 14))
 (segment (start 123.3375 114.75) (end 121.82 114.75) (width 0.2) (layer "B.Cu") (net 14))
 (segment (start 124.6 117.5025) (end 124.6 116.0125) (width 0.2) (layer "B.Cu") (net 14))
 (segment (start 122.91 119.1925) (end 124.6 117.5025) (width 0.2) (layer "B.Cu") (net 14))
 (segment (start 124.6 116.0125) (end 123.3375 114.75) (width 0.2) (layer "B.Cu") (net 14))
 (segment (start 120.21 132.8125) (end 122.91 130.1125) (width 0.2) (layer "B.Cu") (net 14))
 (segment (start 120.21 148.0525) (end 120.21 132.8125) (width 0.2) (layer "B.Cu") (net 14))
 (segment (start 122.91 130.1125) (end 122.91 119.1925) (width 0.2) (layer "B.Cu") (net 14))
 (segment (start 101.09 143.1625) (end 106.525 143.1625) (width 0.2) (layer "F.Cu") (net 13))
 (segment (start 100.865 149.9925) (end 100.865 143.3875) (width 0.2) (layer "F.Cu") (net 13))
 (segment (start 100.865 143.3875) (end 101.09 143.1625) (width 0.2) (layer "F.Cu") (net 13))
 (segment (start 106.525 143.1625) (end 106.615 143.2525) (width 0.2) (layer "F.Cu") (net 13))
 (via (at 106.615 143.2525) (size 0.6) (drill 0.3) (layers "F.Cu" "B.Cu") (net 13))
 (segment (start 120.96 122.5525) (end 121.82 121.6925) (width 0.2) (layer "B.Cu") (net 13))
 (segment (start 114.24 135.6275) (end 114.24 122.5525) (width 0.2) (layer "B.Cu") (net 13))
 (segment (start 106.615 143.2525) (end 114.24 135.6275) (width 0.2) (layer "B.Cu") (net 13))
 (segment (start 114.24 122.5525) (end 120.96 122.5525) (width 0.2) (layer "B.Cu") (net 13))
 (segment (start 121.82 121.6925) (end 121.82 117.29) (width 0.2) (layer "B.Cu") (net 13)))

